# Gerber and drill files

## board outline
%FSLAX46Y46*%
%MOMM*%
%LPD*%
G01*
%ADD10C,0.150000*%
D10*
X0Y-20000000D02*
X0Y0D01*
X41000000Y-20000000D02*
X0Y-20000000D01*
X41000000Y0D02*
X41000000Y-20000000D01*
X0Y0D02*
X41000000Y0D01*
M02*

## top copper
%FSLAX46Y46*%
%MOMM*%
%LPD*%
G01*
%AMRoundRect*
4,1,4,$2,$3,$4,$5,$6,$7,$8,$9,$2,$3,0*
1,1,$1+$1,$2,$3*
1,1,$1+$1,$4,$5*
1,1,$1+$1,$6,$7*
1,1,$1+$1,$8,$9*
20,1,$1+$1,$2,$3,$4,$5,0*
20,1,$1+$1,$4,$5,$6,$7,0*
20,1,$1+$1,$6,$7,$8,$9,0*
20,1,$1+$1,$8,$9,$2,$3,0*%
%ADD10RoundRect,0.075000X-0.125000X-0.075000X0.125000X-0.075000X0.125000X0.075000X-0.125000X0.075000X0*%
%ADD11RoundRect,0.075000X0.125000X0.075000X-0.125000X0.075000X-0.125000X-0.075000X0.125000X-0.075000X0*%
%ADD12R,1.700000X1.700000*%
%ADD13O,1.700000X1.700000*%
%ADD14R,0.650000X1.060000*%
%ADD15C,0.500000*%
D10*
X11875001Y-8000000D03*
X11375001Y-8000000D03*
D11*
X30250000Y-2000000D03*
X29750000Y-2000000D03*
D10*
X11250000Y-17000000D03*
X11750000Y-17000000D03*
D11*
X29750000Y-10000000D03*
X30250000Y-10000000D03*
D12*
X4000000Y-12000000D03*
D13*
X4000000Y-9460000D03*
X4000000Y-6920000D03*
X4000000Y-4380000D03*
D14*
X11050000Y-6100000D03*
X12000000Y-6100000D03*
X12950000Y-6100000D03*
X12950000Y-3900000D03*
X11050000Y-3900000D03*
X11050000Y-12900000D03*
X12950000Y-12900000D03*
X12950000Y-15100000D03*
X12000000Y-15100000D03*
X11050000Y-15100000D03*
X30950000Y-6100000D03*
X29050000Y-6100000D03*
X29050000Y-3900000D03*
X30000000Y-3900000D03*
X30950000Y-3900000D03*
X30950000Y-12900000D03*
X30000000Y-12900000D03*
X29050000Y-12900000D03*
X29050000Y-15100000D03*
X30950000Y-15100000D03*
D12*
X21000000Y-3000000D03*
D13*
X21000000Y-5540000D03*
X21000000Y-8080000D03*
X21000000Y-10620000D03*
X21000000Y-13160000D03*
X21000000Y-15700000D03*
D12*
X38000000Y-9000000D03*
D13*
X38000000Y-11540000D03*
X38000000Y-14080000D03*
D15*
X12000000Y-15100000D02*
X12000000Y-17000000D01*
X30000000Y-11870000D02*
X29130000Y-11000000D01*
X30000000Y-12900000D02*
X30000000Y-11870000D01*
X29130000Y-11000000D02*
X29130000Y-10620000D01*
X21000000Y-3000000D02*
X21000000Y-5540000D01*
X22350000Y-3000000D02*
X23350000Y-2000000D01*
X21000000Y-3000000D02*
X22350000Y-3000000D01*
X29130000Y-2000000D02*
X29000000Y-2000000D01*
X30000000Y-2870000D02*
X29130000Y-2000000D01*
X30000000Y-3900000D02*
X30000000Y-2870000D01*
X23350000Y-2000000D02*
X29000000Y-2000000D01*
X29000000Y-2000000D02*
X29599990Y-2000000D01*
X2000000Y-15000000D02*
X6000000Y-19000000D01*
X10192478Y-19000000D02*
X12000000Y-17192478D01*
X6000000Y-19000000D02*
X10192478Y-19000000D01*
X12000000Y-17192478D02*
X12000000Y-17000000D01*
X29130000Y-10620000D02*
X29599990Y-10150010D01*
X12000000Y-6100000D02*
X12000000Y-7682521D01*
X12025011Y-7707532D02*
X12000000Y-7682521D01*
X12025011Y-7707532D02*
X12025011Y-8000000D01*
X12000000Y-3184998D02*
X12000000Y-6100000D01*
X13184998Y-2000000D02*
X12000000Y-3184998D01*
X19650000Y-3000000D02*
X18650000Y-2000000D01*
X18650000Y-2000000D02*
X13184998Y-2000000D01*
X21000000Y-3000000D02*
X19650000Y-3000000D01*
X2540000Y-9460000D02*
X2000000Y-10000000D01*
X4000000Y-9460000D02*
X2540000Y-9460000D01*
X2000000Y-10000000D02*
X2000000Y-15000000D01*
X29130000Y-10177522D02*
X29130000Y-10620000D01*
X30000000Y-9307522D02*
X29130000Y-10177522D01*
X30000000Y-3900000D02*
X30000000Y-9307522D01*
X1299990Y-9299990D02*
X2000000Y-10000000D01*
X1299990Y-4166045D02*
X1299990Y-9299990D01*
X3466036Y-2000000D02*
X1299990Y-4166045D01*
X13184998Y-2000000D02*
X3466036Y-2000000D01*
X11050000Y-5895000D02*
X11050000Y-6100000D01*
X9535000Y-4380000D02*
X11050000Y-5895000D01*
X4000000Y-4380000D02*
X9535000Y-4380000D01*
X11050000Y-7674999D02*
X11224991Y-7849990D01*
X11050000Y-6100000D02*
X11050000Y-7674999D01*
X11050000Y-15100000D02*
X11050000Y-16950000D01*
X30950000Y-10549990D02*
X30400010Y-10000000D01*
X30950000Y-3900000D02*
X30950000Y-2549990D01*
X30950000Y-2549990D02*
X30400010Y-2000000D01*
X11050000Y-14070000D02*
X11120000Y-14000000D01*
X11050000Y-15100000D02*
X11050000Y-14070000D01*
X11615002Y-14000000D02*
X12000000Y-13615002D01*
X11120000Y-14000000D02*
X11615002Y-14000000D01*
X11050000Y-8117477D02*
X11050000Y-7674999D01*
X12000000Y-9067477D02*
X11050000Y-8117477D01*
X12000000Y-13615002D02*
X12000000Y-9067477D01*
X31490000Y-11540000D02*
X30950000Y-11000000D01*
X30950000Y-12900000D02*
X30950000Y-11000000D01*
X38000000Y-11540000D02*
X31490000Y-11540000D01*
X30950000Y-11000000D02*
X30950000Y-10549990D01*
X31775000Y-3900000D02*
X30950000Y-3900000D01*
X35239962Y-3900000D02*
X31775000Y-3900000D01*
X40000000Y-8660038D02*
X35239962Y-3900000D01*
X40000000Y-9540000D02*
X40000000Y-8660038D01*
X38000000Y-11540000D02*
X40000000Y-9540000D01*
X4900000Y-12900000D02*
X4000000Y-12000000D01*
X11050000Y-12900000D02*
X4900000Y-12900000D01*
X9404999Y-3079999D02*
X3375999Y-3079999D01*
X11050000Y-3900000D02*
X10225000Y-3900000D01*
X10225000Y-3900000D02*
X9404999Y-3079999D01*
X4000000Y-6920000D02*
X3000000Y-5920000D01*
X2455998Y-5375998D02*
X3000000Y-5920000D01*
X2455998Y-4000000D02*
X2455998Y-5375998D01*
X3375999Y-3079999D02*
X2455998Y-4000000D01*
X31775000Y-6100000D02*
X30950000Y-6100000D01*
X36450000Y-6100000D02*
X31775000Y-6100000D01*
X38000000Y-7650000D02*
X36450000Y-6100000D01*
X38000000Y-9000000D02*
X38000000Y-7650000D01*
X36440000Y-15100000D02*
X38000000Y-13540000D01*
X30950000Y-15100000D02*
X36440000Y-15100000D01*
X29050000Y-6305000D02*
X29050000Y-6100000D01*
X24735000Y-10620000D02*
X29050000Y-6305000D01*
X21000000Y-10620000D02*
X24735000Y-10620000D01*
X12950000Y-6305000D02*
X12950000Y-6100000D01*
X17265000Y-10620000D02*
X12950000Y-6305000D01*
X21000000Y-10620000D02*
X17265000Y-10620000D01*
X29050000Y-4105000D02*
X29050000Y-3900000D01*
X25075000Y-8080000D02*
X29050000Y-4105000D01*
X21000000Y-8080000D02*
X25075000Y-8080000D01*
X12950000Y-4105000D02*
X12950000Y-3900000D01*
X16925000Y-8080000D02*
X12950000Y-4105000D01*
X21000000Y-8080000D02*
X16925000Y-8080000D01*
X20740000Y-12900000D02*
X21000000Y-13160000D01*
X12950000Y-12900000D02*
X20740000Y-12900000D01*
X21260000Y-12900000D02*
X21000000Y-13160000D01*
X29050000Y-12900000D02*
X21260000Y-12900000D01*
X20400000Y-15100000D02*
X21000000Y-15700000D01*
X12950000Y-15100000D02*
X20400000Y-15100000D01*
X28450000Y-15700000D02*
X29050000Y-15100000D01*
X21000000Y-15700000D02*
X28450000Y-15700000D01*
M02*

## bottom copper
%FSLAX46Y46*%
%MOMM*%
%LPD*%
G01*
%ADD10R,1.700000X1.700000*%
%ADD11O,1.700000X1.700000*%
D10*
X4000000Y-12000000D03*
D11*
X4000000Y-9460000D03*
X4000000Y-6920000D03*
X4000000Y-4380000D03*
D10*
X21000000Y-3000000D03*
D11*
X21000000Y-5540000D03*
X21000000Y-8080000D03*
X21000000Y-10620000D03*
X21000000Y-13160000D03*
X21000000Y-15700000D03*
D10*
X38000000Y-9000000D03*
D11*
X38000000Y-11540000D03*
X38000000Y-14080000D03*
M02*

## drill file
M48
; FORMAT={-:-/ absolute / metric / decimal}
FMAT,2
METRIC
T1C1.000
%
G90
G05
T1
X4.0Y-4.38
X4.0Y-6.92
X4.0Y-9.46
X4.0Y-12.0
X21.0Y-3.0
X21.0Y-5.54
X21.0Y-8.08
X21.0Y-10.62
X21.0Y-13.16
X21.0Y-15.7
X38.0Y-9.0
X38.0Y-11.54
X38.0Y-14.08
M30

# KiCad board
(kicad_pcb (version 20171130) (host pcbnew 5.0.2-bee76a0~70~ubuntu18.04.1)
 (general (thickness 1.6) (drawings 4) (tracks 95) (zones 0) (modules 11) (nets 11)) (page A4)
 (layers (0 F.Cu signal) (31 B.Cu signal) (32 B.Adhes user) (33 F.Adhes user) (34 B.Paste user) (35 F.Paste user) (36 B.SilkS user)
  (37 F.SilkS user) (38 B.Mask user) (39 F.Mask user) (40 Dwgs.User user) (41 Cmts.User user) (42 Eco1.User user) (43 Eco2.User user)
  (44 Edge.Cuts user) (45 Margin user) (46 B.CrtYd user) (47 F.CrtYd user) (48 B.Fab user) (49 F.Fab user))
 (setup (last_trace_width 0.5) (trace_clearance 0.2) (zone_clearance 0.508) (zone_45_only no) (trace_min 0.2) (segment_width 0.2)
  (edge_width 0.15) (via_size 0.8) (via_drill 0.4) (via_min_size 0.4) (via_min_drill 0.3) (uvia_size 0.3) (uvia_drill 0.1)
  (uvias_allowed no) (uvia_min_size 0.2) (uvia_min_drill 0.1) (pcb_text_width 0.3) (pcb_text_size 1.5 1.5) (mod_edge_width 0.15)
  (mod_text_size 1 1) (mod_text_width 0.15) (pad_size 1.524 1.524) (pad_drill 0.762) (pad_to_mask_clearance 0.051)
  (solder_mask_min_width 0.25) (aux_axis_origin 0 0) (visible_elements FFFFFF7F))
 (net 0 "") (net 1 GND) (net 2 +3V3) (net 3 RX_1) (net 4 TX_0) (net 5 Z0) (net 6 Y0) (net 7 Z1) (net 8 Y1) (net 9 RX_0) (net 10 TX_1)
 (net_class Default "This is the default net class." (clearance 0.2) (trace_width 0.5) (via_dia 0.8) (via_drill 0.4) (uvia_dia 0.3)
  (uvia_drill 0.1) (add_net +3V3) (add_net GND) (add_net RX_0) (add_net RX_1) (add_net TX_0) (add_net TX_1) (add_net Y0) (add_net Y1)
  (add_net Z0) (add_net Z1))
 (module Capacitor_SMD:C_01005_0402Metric (layer F.Cu) (at 11.625001 8)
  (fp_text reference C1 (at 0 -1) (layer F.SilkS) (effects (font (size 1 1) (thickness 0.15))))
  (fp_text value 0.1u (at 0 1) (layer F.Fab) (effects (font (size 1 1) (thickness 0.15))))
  (pad 2 smd roundrect (at 0.25 0) (size 0.4 0.3) (layers F.Cu F.Mask) (roundrect_rratio 0.25) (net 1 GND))
  (pad 1 smd roundrect (at -0.25 0) (size 0.4 0.3) (layers F.Cu F.Mask) (roundrect_rratio 0.25) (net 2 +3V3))
  (pad "" smd roundrect (at 0.275 0) (size 0.27 0.27) (layers F.Paste) (roundrect_rratio 0.25))
  (pad "" smd roundrect (at -0.275 0) (size 0.27 0.27) (layers F.Paste) (roundrect_rratio 0.25)))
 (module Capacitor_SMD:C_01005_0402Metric (layer F.Cu) (at 30 2 180)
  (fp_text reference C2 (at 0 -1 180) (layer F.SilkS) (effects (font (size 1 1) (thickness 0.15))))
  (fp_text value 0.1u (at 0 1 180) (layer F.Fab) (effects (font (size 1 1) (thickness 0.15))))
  (pad "" smd roundrect (at -0.275 0 180) (size 0.27 0.27) (layers F.Paste) (roundrect_rratio 0.25))
  (pad "" smd roundrect (at 0.275 0 180) (size 0.27 0.27) (layers F.Paste) (roundrect_rratio 0.25))
  (pad 1 smd roundrect (at -0.25 0 180) (size 0.4 0.3) (layers F.Cu F.Mask) (roundrect_rratio 0.25) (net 2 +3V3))
  (pad 2 smd roundrect (at 0.25 0 180) (size 0.4 0.3) (layers F.Cu F.Mask) (roundrect_rratio 0.25) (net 1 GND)))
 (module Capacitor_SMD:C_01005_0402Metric (layer F.Cu) (at 11.5 17)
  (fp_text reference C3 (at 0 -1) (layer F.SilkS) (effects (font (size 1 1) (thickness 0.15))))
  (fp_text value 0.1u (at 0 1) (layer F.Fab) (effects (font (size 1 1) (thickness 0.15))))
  (pad "" smd roundrect (at -0.275 0) (size 0.27 0.27) (layers F.Paste) (roundrect_rratio 0.25))
  (pad "" smd roundrect (at 0.275 0) (size 0.27 0.27) (layers F.Paste) (roundrect_rratio 0.25))
  (pad 1 smd roundrect (at -0.25 0) (size 0.4 0.3) (layers F.Cu F.Mask) (roundrect_rratio 0.25) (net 2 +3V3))
  (pad 2 smd roundrect (at 0.25 0) (size 0.4 0.3) (layers F.Cu F.Mask) (roundrect_rratio 0.25) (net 1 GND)))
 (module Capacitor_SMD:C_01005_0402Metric (layer F.Cu) (at 30 10 180)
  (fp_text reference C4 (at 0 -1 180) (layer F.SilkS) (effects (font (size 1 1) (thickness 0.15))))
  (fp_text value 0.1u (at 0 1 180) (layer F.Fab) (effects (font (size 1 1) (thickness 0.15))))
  (pad 2 smd roundrect (at 0.25 0 180) (size 0.4 0.3) (layers F.Cu F.Mask) (roundrect_rratio 0.25) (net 1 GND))
  (pad 1 smd roundrect (at -0.25 0 180) (size 0.4 0.3) (layers F.Cu F.Mask) (roundrect_rratio 0.25) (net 2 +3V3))
  (pad "" smd roundrect (at 0.275 0 180) (size 0.27 0.27) (layers F.Paste) (roundrect_rratio 0.25))
  (pad "" smd roundrect (at -0.275 0 180) (size 0.27 0.27) (layers F.Paste) (roundrect_rratio 0.25)))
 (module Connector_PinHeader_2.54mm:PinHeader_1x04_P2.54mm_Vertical (layer F.Cu) (at 4 12 180)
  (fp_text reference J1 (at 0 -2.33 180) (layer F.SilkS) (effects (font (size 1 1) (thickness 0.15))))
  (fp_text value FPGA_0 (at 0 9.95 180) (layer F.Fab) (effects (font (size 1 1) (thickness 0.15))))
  (pad 1 thru_hole rect (at 0 0 180) (size 1.7 1.7) (drill 1) (layers *.Cu *.Mask) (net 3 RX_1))
  (pad 2 thru_hole oval (at 0 2.54 180) (size 1.7 1.7) (drill 1) (layers *.Cu *.Mask) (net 1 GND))
  (pad 3 thru_hole oval (at 0 5.08 180) (size 1.7 1.7) (drill 1) (layers *.Cu *.Mask) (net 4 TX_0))
  (pad 4 thru_hole oval (at 0 7.62 180) (size 1.7 1.7) (drill 1) (layers *.Cu *.Mask) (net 2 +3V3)))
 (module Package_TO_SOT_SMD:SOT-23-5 (layer F.Cu) (at 12 5 90)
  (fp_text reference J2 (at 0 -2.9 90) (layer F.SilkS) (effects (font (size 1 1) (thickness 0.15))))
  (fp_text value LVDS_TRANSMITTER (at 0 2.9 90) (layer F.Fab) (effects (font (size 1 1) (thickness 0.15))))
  (pad 1 smd rect (at -1.1 -0.95 90) (size 1.06 0.65) (layers F.Cu F.Paste F.Mask) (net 2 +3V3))
  (pad 2 smd rect (at -1.1 0 90) (size 1.06 0.65) (layers F.Cu F.Paste F.Mask) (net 1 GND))
  (pad 3 smd rect (at -1.1 0.95 90) (size 1.06 0.65) (layers F.Cu F.Paste F.Mask) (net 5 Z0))
  (pad 4 smd rect (at 1.1 0.95 90) (size 1.06 0.65) (layers F.Cu F.Paste F.Mask) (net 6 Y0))
  (pad 5 smd rect (at 1.1 -0.95 90) (size 1.06 0.65) (layers F.Cu F.Paste F.Mask) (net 4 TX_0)))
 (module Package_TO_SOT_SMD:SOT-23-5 (layer F.Cu) (at 12 14 90)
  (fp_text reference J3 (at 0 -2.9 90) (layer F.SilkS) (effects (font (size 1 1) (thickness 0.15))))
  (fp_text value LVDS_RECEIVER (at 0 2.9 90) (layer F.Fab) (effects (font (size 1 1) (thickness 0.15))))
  (pad 5 smd rect (at 1.1 -0.95 90) (size 1.06 0.65) (layers F.Cu F.Paste F.Mask) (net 3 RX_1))
  (pad 4 smd rect (at 1.1 0.95 90) (size 1.06 0.65) (layers F.Cu F.Paste F.Mask) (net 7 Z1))
  (pad 3 smd rect (at -1.1 0.95 90) (size 1.06 0.65) (layers F.Cu F.Paste F.Mask) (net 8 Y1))
  (pad 2 smd rect (at -1.1 0 90) (size 1.06 0.65) (layers F.Cu F.Paste F.Mask) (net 1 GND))
  (pad 1 smd rect (at -1.1 -0.95 90) (size 1.06 0.65) (layers F.Cu F.Paste F.Mask) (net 2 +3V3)))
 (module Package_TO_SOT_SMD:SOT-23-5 (layer F.Cu) (at 30 5 270)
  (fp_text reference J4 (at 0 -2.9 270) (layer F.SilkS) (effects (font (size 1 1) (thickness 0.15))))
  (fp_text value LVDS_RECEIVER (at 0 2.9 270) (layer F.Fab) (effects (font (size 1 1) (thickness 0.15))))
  (pad 5 smd rect (at 1.1 -0.95 270) (size 1.06 0.65) (layers F.Cu F.Paste F.Mask) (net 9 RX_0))
  (pad 4 smd rect (at 1.1 0.95 270) (size 1.06 0.65) (layers F.Cu F.Paste F.Mask) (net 5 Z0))
  (pad 3 smd rect (at -1.1 0.95 270) (size 1.06 0.65) (layers F.Cu F.Paste F.Mask) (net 6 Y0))
  (pad 2 smd rect (at -1.1 0 270) (size 1.06 0.65) (layers F.Cu F.Paste F.Mask) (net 1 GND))
  (pad 1 smd rect (at -1.1 -0.95 270) (size 1.06 0.65) (layers F.Cu F.Paste F.Mask) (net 2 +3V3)))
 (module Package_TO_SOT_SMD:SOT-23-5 (layer F.Cu) (at 30 14 270)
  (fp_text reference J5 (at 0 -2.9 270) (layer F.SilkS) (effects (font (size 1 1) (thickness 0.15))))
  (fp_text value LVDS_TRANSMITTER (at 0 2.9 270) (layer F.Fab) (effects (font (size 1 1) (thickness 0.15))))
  (pad 1 smd rect (at -1.1 -0.95 270) (size 1.06 0.65) (layers F.Cu F.Paste F.Mask) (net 2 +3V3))
  (pad 2 smd rect (at -1.1 0 270) (size 1.06 0.65) (layers F.Cu F.Paste F.Mask) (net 1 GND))
  (pad 3 smd rect (at -1.1 0.95 270) (size 1.06 0.65) (layers F.Cu F.Paste F.Mask) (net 7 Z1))
  (pad 4 smd rect (at 1.1 0.95 270) (size 1.06 0.65) (layers F.Cu F.Paste F.Mask) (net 8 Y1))
  (pad 5 smd rect (at 1.1 -0.95 270) (size 1.06 0.65) (layers F.Cu F.Paste F.Mask) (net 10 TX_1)))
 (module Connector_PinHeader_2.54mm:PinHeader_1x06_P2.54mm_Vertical (layer F.Cu) (at 21 3)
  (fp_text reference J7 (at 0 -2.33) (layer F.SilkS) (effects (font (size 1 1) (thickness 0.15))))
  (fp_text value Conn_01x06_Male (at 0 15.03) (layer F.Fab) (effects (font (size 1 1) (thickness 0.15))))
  (pad 1 thru_hole rect (at 0 0) (size 1.7 1.7) (drill 1) (layers *.Cu *.Mask) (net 1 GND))
  (pad 2 thru_hole oval (at 0 2.54) (size 1.7 1.7) (drill 1) (layers *.Cu *.Mask) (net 1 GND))
  (pad 3 thru_hole oval (at 0 5.08) (size 1.7 1.7) (drill 1) (layers *.Cu *.Mask) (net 6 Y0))
  (pad 4 thru_hole oval (at 0 7.62) (size 1.7 1.7) (drill 1) (layers *.Cu *.Mask) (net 5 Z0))
  (pad 5 thru_hole oval (at 0 10.16) (size 1.7 1.7) (drill 1) (layers *.Cu *.Mask) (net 7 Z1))
  (pad 6 thru_hole oval (at 0 12.7) (size 1.7 1.7) (drill 1) (layers *.Cu *.Mask) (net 8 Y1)))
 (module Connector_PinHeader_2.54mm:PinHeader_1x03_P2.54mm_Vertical (layer F.Cu) (at 38 9)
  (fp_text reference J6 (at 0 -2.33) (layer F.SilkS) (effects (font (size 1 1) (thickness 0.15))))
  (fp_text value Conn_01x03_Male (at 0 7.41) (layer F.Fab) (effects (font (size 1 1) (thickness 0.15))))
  (pad 1 thru_hole rect (at 0 0) (size 1.7 1.7) (drill 1) (layers *.Cu *.Mask) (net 9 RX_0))
  (pad 2 thru_hole oval (at 0 2.54) (size 1.7 1.7) (drill 1) (layers *.Cu *.Mask) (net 2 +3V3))
  (pad 3 thru_hole oval (at 0 5.08) (size 1.7 1.7) (drill 1) (layers *.Cu *.Mask) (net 10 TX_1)))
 (gr_line (start 0 20) (end 0 0) (layer Edge.Cuts) (width 0.15))
 (gr_line (start 41 20) (end 0 20) (layer Edge.Cuts) (width 0.15))
 (gr_line (start 41 0) (end 41 20) (layer Edge.Cuts) (width 0.15))
 (gr_line (start 0 0) (end 41 0) (layer Edge.Cuts) (width 0.15))
 (segment (start 12 15.1) (end 12 17) (width 0.5) (layer F.Cu) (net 1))
 (segment (start 30 11.87) (end 29.13 11) (width 0.5) (layer F.Cu) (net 1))
 (segment (start 30 12.9) (end 30 11.87) (width 0.5) (layer F.Cu) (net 1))
 (segment (start 29.13 11) (end 29.13 10.62) (width 0.5) (layer F.Cu) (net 1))
 (segment (start 21 3) (end 21 5.54) (width 0.5) (layer F.Cu) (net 1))
 (segment (start 22.35 3) (end 23.35 2) (width 0.5) (layer F.Cu) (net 1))
 (segment (start 21 3) (end 22.35 3) (width 0.5) (layer F.Cu) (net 1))
 (segment (start 29.13 2) (end 29 2) (width 0.5) (layer F.Cu) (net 1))
 (segment (start 30 2.87) (end 29.13 2) (width 0.5) (layer F.Cu) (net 1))
 (segment (start 30 3.9) (end 30 2.87) (width 0.5) (layer F.Cu) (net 1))
 (segment (start 23.35 2) (end 29 2) (width 0.5) (layer F.Cu) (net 1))
 (segment (start 29 2) (end 29.59999 2) (width 0.5) (layer F.Cu) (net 1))
 (segment (start 2 15) (end 6 19) (width 0.5) (layer F.Cu) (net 1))
 (segment (start 10.192478 19) (end 12 17.192478) (width 0.5) (layer F.Cu) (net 1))
 (segment (start 6 19) (end 10.192478 19) (width 0.5) (layer F.Cu) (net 1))
 (segment (start 12 17.192478) (end 12 17) (width 0.5) (layer F.Cu) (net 1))
 (segment (start 29.13 10.62) (end 29.59999 10.15001) (width 0.5) (layer F.Cu) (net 1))
 (segment (start 12 6.1) (end 12 7.682521) (width 0.5) (layer F.Cu) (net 1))
 (segment (start 12.025011 7.707532) (end 12 7.682521) (width 0.5) (layer F.Cu) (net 1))
 (segment (start 12.025011 7.707532) (end 12.025011 8) (width 0.5) (layer F.Cu) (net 1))
 (segment (start 12 3.184998) (end 12 6.1) (width 0.5) (layer F.Cu) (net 1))
 (segment (start 13.184998 2) (end 12 3.184998) (width 0.5) (layer F.Cu) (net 1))
 (segment (start 19.65 3) (end 18.65 2) (width 0.5) (layer F.Cu) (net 1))
 (segment (start 18.65 2) (end 13.184998 2) (width 0.5) (layer F.Cu) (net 1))
 (segment (start 21 3) (end 19.65 3) (width 0.5) (layer F.Cu) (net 1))
 (segment (start 2.54 9.46) (end 2 10) (width 0.5) (layer F.Cu) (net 1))
 (segment (start 4 9.46) (end 2.54 9.46) (width 0.5) (layer F.Cu) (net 1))
 (segment (start 2 10) (end 2 15) (width 0.5) (layer F.Cu) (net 1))
 (segment (start 29.13 10.177522) (end 29.13 10.62) (width 0.5) (layer F.Cu) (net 1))
 (segment (start 30 9.307522) (end 29.13 10.177522) (width 0.5) (layer F.Cu) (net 1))
 (segment (start 30 3.9) (end 30 9.307522) (width 0.5) (layer F.Cu) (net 1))
 (segment (start 1.29999 9.29999) (end 2 10) (width 0.5) (layer F.Cu) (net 1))
 (segment (start 1.29999 4.166045) (end 1.29999 9.29999) (width 0.5) (layer F.Cu) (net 1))
 (segment (start 3.466036 2) (end 1.29999 4.166045) (width 0.5) (layer F.Cu) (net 1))
 (segment (start 13.184998 2) (end 3.466036 2) (width 0.5) (layer F.Cu) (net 1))
 (segment (start 11.05 5.895) (end 11.05 6.1) (width 0.5) (layer F.Cu) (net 2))
 (segment (start 9.535 4.38) (end 11.05 5.895) (width 0.5) (layer F.Cu) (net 2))
 (segment (start 4 4.38) (end 9.535 4.38) (width 0.5) (layer F.Cu) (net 2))
 (segment (start 11.05 7.674999) (end 11.224991 7.84999) (width 0.5) (layer F.Cu) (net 2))
 (segment (start 11.05 6.1) (end 11.05 7.674999) (width 0.5) (layer F.Cu) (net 2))
 (segment (start 11.05 15.1) (end 11.05 16.95) (width 0.5) (layer F.Cu) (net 2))
 (segment (start 30.95 10.54999) (end 30.40001 10) (width 0.5) (layer F.Cu) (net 2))
 (segment (start 30.95 3.9) (end 30.95 2.54999) (width 0.5) (layer F.Cu) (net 2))
 (segment (start 30.95 2.54999) (end 30.40001 2) (width 0.5) (layer F.Cu) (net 2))
 (segment (start 11.05 14.07) (end 11.12 14) (width 0.5) (layer F.Cu) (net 2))
 (segment (start 11.05 15.1) (end 11.05 14.07) (width 0.5) (layer F.Cu) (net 2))
 (segment (start 11.615002 14) (end 12 13.615002) (width 0.5) (layer F.Cu) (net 2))
 (segment (start 11.12 14) (end 11.615002 14) (width 0.5) (layer F.Cu) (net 2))
 (segment (start 11.05 8.117477) (end 11.05 7.674999) (width 0.5) (layer F.Cu) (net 2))
 (segment (start 12 9.067477) (end 11.05 8.117477) (width 0.5) (layer F.Cu) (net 2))
 (segment (start 12 13.615002) (end 12 9.067477) (width 0.5) (layer F.Cu) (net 2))
 (segment (start 31.49 11.54) (end 30.95 11) (width 0.5) (layer F.Cu) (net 2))
 (segment (start 30.95 12.9) (end 30.95 11) (width 0.5) (layer F.Cu) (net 2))
 (segment (start 38 11.54) (end 31.49 11.54) (width 0.5) (layer F.Cu) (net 2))
 (segment (start 30.95 11) (end 30.95 10.54999) (width 0.5) (layer F.Cu) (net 2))
 (segment (start 31.775 3.9) (end 30.95 3.9) (width 0.5) (layer F.Cu) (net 2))
 (segment (start 35.239962 3.9) (end 31.775 3.9) (width 0.5) (layer F.Cu) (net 2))
 (segment (start 40 8.660038) (end 35.239962 3.9) (width 0.5) (layer F.Cu) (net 2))
 (segment (start 40 9.54) (end 40 8.660038) (width 0.5) (layer F.Cu) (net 2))
 (segment (start 38 11.54) (end 40 9.54) (width 0.5) (layer F.Cu) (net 2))
 (segment (start 4.9 12.9) (end 4 12) (width 0.5) (layer F.Cu) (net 3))
 (segment (start 11.05 12.9) (end 4.9 12.9) (width 0.5) (layer F.Cu) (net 3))
 (segment (start 9.404999 3.079999) (end 3.375999 3.079999) (width 0.5) (layer F.Cu) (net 4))
 (segment (start 11.05 3.9) (end 10.225 3.9) (width 0.5) (layer F.Cu) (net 4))
 (segment (start 10.225 3.9) (end 9.404999 3.079999) (width 0.5) (layer F.Cu) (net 4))
 (segment (start 4 6.92) (end 3 5.92) (width 0.5) (layer F.Cu) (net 4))
 (segment (start 2.455998 5.375998) (end 3 5.92) (width 0.5) (layer F.Cu) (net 4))
 (segment (start 2.455998 4) (end 2.455998 5.375998) (width 0.5) (layer F.Cu) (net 4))
 (segment (start 3.375999 3.079999) (end 2.455998 4) (width 0.5) (layer F.Cu) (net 4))
 (segment (start 31.775 6.1) (end 30.95 6.1) (width 0.5) (layer F.Cu) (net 9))
 (segment (start 36.45 6.1) (end 31.775 6.1) (width 0.5) (layer F.Cu) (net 9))
 (segment (start 38 7.65) (end 36.45 6.1) (width 0.5) (layer F.Cu) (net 9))
 (segment (start 38 9) (end 38 7.65) (width 0.5) (layer F.Cu) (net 9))
 (segment (start 36.44 15.1) (end 38 13.54) (width 0.5) (layer F.Cu) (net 10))
 (segment (start 30.95 15.1) (end 36.44 15.1) (width 0.5) (layer F.Cu) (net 10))
 (segment (start 29.05 6.305) (end 29.05 6.1) (width 0.5) (layer F.Cu) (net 5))
 (segment (start 24.735 10.62) (end 29.05 6.305) (width 0.5) (layer F.Cu) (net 5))
 (segment (start 21 10.62) (end 24.735 10.62) (width 0.5) (layer F.Cu) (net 5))
 (segment (start 12.95 6.305) (end 12.95 6.1) (width 0.5) (layer F.Cu) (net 5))
 (segment (start 17.265 10.62) (end 12.95 6.305) (width 0.5) (layer F.Cu) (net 5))
 (segment (start 21 10.62) (end 17.265 10.62) (width 0.5) (layer F.Cu) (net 5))
 (segment (start 29.05 4.105) (end 29.05 3.9) (width 0.5) (layer F.Cu) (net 6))
 (segment (start 25.075 8.08) (end 29.05 4.105) (width 0.5) (layer F.Cu) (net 6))
 (segment (start 21 8.08) (end 25.075 8.08) (width 0.5) (layer F.Cu) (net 6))
 (segment (start 12.95 4.105) (end 12.95 3.9) (width 0.5) (layer F.Cu) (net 6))
 (segment (start 16.925 8.08) (end 12.95 4.105) (width 0.5) (layer F.Cu) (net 6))
 (segment (start 21 8.08) (end 16.925 8.08) (width 0.5) (layer F.Cu) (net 6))
 (segment (start 20.74 12.9) (end 21 13.16) (width 0.5) (layer F.Cu) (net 7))
 (segment (start 12.95 12.9) (end 20.74 12.9) (width 0.5) (layer F.Cu) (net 7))
 (segment (start 21.26 12.9) (end 21 13.16) (width 0.5) (layer F.Cu) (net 7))
 (segment (start 29.05 12.9) (end 21.26 12.9) (width 0.5) (layer F.Cu) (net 7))
 (segment (start 20.4 15.1) (end 21 15.7) (width 0.5) (layer F.Cu) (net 8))
 (segment (start 12.95 15.1) (end 20.4 15.1) (width 0.5) (layer F.Cu) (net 8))
 (segment (start 28.45 15.7) (end 29.05 15.1) (width 0.5) (layer F.Cu) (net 8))
 (segment (start 21 15.7) (end 28.45 15.7) (width 0.5) (layer F.Cu) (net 8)))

